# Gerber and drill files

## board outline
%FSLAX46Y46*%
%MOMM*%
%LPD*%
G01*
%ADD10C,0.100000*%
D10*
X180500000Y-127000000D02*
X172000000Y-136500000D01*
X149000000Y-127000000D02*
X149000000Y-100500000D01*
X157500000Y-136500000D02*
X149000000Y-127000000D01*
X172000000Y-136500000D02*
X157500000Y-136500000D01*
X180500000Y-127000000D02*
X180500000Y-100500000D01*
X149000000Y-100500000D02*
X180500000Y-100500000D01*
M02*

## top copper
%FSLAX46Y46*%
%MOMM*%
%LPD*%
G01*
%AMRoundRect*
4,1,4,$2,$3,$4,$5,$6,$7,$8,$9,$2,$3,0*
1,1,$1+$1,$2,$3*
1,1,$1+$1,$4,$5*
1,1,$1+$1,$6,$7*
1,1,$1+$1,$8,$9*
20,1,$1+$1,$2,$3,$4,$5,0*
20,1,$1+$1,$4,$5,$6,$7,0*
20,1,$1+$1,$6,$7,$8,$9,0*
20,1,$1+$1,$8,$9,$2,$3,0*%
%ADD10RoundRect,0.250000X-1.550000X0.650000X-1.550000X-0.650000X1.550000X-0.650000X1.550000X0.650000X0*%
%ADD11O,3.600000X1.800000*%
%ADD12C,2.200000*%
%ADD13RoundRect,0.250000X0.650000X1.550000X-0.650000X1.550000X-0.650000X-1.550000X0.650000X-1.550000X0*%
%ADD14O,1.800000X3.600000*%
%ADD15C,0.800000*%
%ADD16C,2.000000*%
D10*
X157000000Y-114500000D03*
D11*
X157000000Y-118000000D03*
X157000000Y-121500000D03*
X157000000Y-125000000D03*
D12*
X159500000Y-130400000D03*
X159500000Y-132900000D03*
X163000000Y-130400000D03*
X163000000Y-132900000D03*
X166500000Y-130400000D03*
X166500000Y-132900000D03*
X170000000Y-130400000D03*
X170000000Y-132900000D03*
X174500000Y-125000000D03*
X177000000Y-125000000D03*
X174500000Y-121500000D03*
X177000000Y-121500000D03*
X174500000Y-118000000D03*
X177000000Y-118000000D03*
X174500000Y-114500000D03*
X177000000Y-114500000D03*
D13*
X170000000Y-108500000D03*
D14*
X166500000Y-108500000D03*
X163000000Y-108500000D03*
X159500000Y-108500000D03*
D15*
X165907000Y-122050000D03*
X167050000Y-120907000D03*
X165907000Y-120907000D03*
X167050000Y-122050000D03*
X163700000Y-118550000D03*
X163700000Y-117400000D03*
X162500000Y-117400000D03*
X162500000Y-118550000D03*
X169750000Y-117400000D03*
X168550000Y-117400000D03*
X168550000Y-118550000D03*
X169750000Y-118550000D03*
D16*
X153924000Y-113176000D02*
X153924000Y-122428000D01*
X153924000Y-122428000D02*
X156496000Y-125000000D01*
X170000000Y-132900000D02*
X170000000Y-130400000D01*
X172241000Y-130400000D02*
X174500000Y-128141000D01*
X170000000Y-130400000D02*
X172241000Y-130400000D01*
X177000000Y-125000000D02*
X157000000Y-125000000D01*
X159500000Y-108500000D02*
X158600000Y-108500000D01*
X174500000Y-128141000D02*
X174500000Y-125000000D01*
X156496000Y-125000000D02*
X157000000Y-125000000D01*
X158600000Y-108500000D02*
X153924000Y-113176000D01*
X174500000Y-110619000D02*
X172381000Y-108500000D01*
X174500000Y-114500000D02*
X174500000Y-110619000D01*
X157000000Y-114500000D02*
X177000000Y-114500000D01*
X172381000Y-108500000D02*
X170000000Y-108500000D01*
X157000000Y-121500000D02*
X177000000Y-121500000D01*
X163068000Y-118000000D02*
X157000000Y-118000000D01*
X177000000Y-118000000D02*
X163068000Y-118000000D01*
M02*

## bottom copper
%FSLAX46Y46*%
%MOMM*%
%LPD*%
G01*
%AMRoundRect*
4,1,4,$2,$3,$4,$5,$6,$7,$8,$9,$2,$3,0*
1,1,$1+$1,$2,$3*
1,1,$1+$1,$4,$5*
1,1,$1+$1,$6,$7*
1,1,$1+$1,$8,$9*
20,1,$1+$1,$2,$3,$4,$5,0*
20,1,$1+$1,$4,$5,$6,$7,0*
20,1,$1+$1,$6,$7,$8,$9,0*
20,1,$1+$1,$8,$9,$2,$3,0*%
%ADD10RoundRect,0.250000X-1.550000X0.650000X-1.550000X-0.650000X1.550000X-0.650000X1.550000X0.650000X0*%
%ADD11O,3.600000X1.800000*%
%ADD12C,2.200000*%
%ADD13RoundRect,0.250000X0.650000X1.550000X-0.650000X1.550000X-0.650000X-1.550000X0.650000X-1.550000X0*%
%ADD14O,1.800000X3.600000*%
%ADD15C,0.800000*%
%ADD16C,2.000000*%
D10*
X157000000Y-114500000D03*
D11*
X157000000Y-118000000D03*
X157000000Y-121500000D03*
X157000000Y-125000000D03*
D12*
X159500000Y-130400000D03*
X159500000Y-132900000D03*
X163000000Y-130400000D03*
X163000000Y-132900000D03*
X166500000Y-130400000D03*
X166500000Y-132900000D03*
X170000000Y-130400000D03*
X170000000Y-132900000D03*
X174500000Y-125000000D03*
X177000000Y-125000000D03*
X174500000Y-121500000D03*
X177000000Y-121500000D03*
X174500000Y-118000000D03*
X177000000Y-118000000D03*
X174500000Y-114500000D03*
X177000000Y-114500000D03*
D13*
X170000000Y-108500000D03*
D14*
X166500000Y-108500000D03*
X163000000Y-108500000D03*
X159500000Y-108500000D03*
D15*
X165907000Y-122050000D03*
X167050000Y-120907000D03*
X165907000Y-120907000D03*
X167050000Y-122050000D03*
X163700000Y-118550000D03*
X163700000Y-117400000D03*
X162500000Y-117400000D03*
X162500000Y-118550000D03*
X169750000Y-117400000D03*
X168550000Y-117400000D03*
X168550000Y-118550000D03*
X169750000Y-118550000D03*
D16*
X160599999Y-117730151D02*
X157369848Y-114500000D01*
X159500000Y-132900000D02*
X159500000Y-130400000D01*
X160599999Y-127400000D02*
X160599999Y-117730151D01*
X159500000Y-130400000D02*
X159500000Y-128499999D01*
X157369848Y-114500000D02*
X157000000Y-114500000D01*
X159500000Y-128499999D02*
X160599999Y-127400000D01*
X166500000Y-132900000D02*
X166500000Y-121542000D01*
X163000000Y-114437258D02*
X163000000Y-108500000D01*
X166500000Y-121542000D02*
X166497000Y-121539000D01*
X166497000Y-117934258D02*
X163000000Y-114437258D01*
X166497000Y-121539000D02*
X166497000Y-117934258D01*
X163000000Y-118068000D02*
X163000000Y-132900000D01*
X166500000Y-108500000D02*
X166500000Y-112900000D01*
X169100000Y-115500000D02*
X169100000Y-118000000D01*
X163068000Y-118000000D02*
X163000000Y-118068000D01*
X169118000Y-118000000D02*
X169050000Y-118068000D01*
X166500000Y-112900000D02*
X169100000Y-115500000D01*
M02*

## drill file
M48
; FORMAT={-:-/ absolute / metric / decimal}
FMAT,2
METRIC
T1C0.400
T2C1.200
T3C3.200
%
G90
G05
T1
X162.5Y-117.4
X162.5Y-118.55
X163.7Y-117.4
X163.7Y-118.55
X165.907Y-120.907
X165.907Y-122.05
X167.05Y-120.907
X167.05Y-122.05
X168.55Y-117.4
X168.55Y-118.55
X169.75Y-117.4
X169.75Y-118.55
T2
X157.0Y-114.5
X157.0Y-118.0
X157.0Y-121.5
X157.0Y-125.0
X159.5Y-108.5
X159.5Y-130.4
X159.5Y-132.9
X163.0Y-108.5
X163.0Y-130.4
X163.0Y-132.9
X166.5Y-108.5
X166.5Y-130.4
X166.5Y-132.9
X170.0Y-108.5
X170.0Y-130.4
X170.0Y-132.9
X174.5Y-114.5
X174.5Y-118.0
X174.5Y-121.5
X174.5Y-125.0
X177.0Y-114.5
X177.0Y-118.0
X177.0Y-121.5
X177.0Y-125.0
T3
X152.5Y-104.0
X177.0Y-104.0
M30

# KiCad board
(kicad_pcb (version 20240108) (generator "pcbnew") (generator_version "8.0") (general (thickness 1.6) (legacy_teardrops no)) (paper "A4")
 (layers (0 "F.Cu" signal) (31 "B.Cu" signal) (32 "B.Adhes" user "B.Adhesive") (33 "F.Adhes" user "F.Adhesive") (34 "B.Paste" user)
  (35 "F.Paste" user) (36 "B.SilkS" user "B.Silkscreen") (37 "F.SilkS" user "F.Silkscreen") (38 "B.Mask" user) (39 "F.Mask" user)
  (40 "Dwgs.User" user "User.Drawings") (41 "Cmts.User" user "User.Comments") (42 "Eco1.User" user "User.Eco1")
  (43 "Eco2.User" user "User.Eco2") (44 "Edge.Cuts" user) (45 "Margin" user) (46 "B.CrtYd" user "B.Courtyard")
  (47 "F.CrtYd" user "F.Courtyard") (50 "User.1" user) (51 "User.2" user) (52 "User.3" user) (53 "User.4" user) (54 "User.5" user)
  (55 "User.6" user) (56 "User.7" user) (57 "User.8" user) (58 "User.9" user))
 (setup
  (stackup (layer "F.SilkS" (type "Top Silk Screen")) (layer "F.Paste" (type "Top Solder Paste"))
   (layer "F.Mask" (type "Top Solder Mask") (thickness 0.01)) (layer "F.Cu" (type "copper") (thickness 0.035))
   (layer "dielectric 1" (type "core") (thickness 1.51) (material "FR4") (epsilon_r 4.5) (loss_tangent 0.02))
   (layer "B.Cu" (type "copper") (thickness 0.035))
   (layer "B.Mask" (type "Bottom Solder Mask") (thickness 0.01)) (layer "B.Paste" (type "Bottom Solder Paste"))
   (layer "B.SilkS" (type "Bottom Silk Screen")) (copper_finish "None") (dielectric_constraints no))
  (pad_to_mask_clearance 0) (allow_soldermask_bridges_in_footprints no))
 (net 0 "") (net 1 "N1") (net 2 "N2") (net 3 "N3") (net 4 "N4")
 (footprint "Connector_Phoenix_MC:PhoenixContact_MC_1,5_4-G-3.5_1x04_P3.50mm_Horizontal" (layer "F.Cu") (at 157 114.5 -90)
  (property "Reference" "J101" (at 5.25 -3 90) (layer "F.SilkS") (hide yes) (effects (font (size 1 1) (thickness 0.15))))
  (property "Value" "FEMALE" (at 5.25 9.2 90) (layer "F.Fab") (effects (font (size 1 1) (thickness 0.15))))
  (pad "1" thru_hole roundrect (at 0 0 270) (size 1.8 3.6) (drill 1.2) (layers "*.Cu" "*.Mask") (remove_unused_layers no)
   (roundrect_rratio 0.138889) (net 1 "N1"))
  (pad "2" thru_hole oval (at 3.5 0 270) (size 1.8 3.6) (drill 1.2) (layers "*.Cu" "*.Mask") (remove_unused_layers no) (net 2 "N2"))
  (pad "3" thru_hole oval (at 7 0 270) (size 1.8 3.6) (drill 1.2) (layers "*.Cu" "*.Mask") (remove_unused_layers no) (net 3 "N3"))
  (pad "4" thru_hole oval (at 10.5 0 270) (size 1.8 3.6) (drill 1.2) (layers "*.Cu" "*.Mask") (remove_unused_layers no) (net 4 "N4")))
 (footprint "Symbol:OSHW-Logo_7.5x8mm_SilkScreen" (layer "F.Cu") (at 165.227 118.237)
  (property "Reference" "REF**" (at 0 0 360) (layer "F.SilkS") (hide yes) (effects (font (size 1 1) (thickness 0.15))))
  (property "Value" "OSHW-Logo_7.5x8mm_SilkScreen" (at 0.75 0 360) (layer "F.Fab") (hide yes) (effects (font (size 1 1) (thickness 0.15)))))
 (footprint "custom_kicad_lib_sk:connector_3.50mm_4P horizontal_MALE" (layer "F.Cu") (at 164.75 130.4)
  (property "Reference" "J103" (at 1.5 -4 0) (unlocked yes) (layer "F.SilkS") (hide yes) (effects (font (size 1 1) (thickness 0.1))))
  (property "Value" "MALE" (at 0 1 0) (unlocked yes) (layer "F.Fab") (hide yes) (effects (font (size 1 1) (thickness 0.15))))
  (pad "1" thru_hole circle (at -5.25 0) (size 2.2 2.2) (drill 1.2) (layers "*.Cu" "*.Mask") (remove_unused_layers no) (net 1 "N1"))
  (pad "1" thru_hole circle (at -5.25 2.5) (size 2.2 2.2) (drill 1.2) (layers "*.Cu" "*.Mask") (remove_unused_layers no) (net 1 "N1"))
  (pad "2" thru_hole circle (at -1.75 0) (size 2.2 2.2) (drill 1.2) (layers "*.Cu" "*.Mask") (remove_unused_layers no) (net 2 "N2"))
  (pad "2" thru_hole circle (at -1.75 2.5) (size 2.2 2.2) (drill 1.2) (layers "*.Cu" "*.Mask") (remove_unused_layers no) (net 2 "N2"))
  (pad "3" thru_hole circle (at 1.75 0) (size 2.2 2.2) (drill 1.2) (layers "*.Cu" "*.Mask") (remove_unused_layers no) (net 3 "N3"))
  (pad "3" thru_hole circle (at 1.75 2.5) (size 2.2 2.2) (drill 1.2) (layers "*.Cu" "*.Mask") (remove_unused_layers no) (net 3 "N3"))
  (pad "4" thru_hole circle (at 5.25 0) (size 2.2 2.2) (drill 1.2) (layers "*.Cu" "*.Mask") (remove_unused_layers no) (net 4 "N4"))
  (pad "4" thru_hole circle (at 5.25 2.5) (size 2.2 2.2) (drill 1.2) (layers "*.Cu" "*.Mask") (remove_unused_layers no) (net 4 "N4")))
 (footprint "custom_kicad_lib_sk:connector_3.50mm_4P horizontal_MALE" (layer "F.Cu") (at 174.5 119.75 90)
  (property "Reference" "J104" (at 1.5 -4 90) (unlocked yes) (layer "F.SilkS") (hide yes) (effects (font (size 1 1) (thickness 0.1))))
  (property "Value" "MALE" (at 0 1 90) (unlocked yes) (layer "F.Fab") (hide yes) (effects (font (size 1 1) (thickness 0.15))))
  (pad "1" thru_hole circle (at -5.25 0 90) (size 2.2 2.2) (drill 1.2) (layers "*.Cu" "*.Mask") (remove_unused_layers no) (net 4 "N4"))
  (pad "1" thru_hole circle (at -5.25 2.5 90) (size 2.2 2.2) (drill 1.2) (layers "*.Cu" "*.Mask") (remove_unused_layers no) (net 4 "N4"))
  (pad "2" thru_hole circle (at -1.75 0 90) (size 2.2 2.2) (drill 1.2) (layers "*.Cu" "*.Mask") (remove_unused_layers no) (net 3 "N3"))
  (pad "2" thru_hole circle (at -1.75 2.5 90) (size 2.2 2.2) (drill 1.2) (layers "*.Cu" "*.Mask") (remove_unused_layers no) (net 3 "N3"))
  (pad "3" thru_hole circle (at 1.75 0 90) (size 2.2 2.2) (drill 1.2) (layers "*.Cu" "*.Mask") (remove_unused_layers no) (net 2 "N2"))
  (pad "3" thru_hole circle (at 1.75 2.5 90) (size 2.2 2.2) (drill 1.2) (layers "*.Cu" "*.Mask") (remove_unused_layers no) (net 2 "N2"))
  (pad "4" thru_hole circle (at 5.25 0 90) (size 2.2 2.2) (drill 1.2) (layers "*.Cu" "*.Mask") (remove_unused_layers no) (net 1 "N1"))
  (pad "4" thru_hole circle (at 5.25 2.5 90) (size 2.2 2.2) (drill 1.2) (layers "*.Cu" "*.Mask") (remove_unused_layers no) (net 1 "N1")))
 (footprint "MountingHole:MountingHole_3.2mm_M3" (layer "F.Cu") (at 152.5 104)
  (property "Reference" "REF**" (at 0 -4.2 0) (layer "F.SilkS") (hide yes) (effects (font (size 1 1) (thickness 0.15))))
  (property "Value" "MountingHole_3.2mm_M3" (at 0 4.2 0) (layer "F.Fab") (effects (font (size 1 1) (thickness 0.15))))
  (pad "" np_thru_hole circle (at 0 0) (size 3.2 3.2) (drill 3.2) (layers "*.Cu" "*.Mask")))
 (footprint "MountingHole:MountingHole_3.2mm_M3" (layer "F.Cu") (at 177 104)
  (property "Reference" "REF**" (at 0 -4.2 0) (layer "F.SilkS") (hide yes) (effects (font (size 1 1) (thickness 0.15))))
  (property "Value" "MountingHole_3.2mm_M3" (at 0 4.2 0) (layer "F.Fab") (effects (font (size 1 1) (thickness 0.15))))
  (pad "" np_thru_hole circle (at 0 0) (size 3.2 3.2) (drill 3.2) (layers "F&B.Cu" "*.Mask")))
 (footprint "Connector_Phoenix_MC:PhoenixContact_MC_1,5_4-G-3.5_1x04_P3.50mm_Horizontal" (layer "F.Cu") (at 170 108.5 180)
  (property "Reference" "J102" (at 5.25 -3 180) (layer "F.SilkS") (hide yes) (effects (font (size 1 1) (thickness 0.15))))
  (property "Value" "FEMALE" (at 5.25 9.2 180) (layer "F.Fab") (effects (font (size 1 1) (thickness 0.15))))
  (pad "1" thru_hole roundrect (at 0 0 180) (size 1.8 3.6) (drill 1.2) (layers "*.Cu" "*.Mask") (remove_unused_layers no)
   (roundrect_rratio 0.138889) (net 1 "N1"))
  (pad "2" thru_hole oval (at 3.5 0 180) (size 1.8 3.6) (drill 1.2) (layers "*.Cu" "*.Mask") (remove_unused_layers no) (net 2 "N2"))
  (pad "3" thru_hole oval (at 7 0 180) (size 1.8 3.6) (drill 1.2) (layers "*.Cu" "*.Mask") (remove_unused_layers no) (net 3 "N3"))
  (pad "4" thru_hole oval (at 10.5 0 180) (size 1.8 3.6) (drill 1.2) (layers "*.Cu" "*.Mask") (remove_unused_layers no) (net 4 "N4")))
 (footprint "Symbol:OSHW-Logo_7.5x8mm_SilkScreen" (layer "B.Cu") (at 164.973 118.491 180)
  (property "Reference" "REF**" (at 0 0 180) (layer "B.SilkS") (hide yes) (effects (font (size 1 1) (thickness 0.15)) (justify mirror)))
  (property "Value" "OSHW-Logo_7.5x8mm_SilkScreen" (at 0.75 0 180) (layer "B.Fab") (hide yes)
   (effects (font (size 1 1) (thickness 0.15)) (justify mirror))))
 (gr_line (start 180.5 127) (end 172 136.5) (stroke (width 0.1) (type default)) (layer "Edge.Cuts"))
 (gr_line (start 149 127) (end 149 100.5) (stroke (width 0.1) (type default)) (layer "Edge.Cuts"))
 (gr_line (start 157.5 136.5) (end 149 127) (stroke (width 0.1) (type default)) (layer "Edge.Cuts"))
 (gr_line (start 172 136.5) (end 157.5 136.5) (stroke (width 0.1) (type default)) (layer "Edge.Cuts"))
 (gr_line (start 180.5 127) (end 180.5 100.5) (stroke (width 0.1) (type default)) (layer "Edge.Cuts"))
 (gr_line (start 149 100.5) (end 180.5 100.5) (stroke (width 0.1) (type default)) (layer "Edge.Cuts"))
 (segment (start 153.924 113.176) (end 153.924 122.428) (width 2) (layer "F.Cu") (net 4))
 (segment (start 153.924 122.428) (end 156.496 125) (width 2) (layer "F.Cu") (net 4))
 (segment (start 170 132.9) (end 170 130.4) (width 2) (layer "F.Cu") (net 4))
 (segment (start 172.241 130.4) (end 174.5 128.141) (width 2) (layer "F.Cu") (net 4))
 (segment (start 170 130.4) (end 172.241 130.4) (width 2) (layer "F.Cu") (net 4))
 (segment (start 177 125) (end 157 125) (width 2) (layer "F.Cu") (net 4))
 (segment (start 159.5 108.5) (end 158.6 108.5) (width 2) (layer "F.Cu") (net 4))
 (segment (start 174.5 128.141) (end 174.5 125) (width 2) (layer "F.Cu") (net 4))
 (segment (start 156.496 125) (end 157 125) (width 2) (layer "F.Cu") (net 4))
 (segment (start 158.6 108.5) (end 153.924 113.176) (width 2) (layer "F.Cu") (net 4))
 (segment (start 174.5 110.619) (end 172.381 108.5) (width 2) (layer "F.Cu") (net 1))
 (segment (start 174.5 114.5) (end 174.5 110.619) (width 2) (layer "F.Cu") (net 1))
 (segment (start 157 114.5) (end 177 114.5) (width 2) (layer "F.Cu") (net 1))
 (segment (start 172.381 108.5) (end 170 108.5) (width 2) (layer "F.Cu") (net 1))
 (segment (start 160.599999 117.730151) (end 157.369848 114.5) (width 2) (layer "B.Cu") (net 1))
 (segment (start 159.5 132.9) (end 159.5 130.4) (width 2) (layer "B.Cu") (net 1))
 (segment (start 160.599999 127.4) (end 160.599999 117.730151) (width 2) (layer "B.Cu") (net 1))
 (segment (start 159.5 130.4) (end 159.5 128.499999) (width 2) (layer "B.Cu") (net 1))
 (segment (start 157.369848 114.5) (end 157 114.5) (width 2) (layer "B.Cu") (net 1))
 (segment (start 159.5 128.499999) (end 160.599999 127.4) (width 2) (layer "B.Cu") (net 1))
 (segment (start 157 121.5) (end 177 121.5) (width 2) (layer "F.Cu") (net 3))
 (via (at 165.907 122.05) (size 0.8) (drill 0.4) (layers "F.Cu" "B.Cu") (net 3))
 (via (at 167.05 120.907) (size 0.8) (drill 0.4) (layers "F.Cu" "B.Cu") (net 3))
 (via (at 165.907 120.907) (size 0.8) (drill 0.4) (layers "F.Cu" "B.Cu") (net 3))
 (via (at 167.05 122.05) (size 0.8) (drill 0.4) (layers "F.Cu" "B.Cu") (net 3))
 (segment (start 166.5 132.9) (end 166.5 121.542) (width 2) (layer "B.Cu") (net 3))
 (segment (start 163 114.437258) (end 163 108.5) (width 2) (layer "B.Cu") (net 3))
 (segment (start 166.5 121.542) (end 166.497 121.539) (width 2) (layer "B.Cu") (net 3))
 (segment (start 166.497 117.934258) (end 163 114.437258) (width 2) (layer "B.Cu") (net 3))
 (segment (start 166.497 121.539) (end 166.497 117.934258) (width 2) (layer "B.Cu") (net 3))
 (segment (start 163.068 118) (end 157 118) (width 2) (layer "F.Cu") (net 2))
 (segment (start 177 118) (end 163.068 118) (width 2) (layer "F.Cu") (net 2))
 (via (at 163.7 118.55) (size 0.8) (drill 0.4) (layers "F.Cu" "B.Cu") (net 2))
 (via (at 163.7 117.4) (size 0.8) (drill 0.4) (layers "F.Cu" "B.Cu") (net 2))
 (via (at 162.5 117.4) (size 0.8) (drill 0.4) (layers "F.Cu" "B.Cu") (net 2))
 (via (at 162.5 118.55) (size 0.8) (drill 0.4) (layers "F.Cu" "B.Cu") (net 2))
 (via (at 169.75 117.4) (size 0.8) (drill 0.4) (layers "F.Cu" "B.Cu") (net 2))
 (via (at 168.55 117.4) (size 0.8) (drill 0.4) (layers "F.Cu" "B.Cu") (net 2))
 (via (at 168.55 118.55) (size 0.8) (drill 0.4) (layers "F.Cu" "B.Cu") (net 2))
 (via (at 169.75 118.55) (size 0.8) (drill 0.4) (layers "F.Cu" "B.Cu") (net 2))
 (segment (start 163 118.068) (end 163 132.9) (width 2) (layer "B.Cu") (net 2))
 (segment (start 166.5 108.5) (end 166.5 112.9) (width 2) (layer "B.Cu") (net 2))
 (segment (start 169.1 115.5) (end 169.1 118) (width 2) (layer "B.Cu") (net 2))
 (segment (start 163.068 118) (end 163 118.068) (width 2) (layer "B.Cu") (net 2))
 (segment (start 169.118 118) (end 169.05 118.068) (width 2) (layer "B.Cu") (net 2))
 (segment (start 166.5 112.9) (end 169.1 115.5) (width 2) (layer "B.Cu") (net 2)))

